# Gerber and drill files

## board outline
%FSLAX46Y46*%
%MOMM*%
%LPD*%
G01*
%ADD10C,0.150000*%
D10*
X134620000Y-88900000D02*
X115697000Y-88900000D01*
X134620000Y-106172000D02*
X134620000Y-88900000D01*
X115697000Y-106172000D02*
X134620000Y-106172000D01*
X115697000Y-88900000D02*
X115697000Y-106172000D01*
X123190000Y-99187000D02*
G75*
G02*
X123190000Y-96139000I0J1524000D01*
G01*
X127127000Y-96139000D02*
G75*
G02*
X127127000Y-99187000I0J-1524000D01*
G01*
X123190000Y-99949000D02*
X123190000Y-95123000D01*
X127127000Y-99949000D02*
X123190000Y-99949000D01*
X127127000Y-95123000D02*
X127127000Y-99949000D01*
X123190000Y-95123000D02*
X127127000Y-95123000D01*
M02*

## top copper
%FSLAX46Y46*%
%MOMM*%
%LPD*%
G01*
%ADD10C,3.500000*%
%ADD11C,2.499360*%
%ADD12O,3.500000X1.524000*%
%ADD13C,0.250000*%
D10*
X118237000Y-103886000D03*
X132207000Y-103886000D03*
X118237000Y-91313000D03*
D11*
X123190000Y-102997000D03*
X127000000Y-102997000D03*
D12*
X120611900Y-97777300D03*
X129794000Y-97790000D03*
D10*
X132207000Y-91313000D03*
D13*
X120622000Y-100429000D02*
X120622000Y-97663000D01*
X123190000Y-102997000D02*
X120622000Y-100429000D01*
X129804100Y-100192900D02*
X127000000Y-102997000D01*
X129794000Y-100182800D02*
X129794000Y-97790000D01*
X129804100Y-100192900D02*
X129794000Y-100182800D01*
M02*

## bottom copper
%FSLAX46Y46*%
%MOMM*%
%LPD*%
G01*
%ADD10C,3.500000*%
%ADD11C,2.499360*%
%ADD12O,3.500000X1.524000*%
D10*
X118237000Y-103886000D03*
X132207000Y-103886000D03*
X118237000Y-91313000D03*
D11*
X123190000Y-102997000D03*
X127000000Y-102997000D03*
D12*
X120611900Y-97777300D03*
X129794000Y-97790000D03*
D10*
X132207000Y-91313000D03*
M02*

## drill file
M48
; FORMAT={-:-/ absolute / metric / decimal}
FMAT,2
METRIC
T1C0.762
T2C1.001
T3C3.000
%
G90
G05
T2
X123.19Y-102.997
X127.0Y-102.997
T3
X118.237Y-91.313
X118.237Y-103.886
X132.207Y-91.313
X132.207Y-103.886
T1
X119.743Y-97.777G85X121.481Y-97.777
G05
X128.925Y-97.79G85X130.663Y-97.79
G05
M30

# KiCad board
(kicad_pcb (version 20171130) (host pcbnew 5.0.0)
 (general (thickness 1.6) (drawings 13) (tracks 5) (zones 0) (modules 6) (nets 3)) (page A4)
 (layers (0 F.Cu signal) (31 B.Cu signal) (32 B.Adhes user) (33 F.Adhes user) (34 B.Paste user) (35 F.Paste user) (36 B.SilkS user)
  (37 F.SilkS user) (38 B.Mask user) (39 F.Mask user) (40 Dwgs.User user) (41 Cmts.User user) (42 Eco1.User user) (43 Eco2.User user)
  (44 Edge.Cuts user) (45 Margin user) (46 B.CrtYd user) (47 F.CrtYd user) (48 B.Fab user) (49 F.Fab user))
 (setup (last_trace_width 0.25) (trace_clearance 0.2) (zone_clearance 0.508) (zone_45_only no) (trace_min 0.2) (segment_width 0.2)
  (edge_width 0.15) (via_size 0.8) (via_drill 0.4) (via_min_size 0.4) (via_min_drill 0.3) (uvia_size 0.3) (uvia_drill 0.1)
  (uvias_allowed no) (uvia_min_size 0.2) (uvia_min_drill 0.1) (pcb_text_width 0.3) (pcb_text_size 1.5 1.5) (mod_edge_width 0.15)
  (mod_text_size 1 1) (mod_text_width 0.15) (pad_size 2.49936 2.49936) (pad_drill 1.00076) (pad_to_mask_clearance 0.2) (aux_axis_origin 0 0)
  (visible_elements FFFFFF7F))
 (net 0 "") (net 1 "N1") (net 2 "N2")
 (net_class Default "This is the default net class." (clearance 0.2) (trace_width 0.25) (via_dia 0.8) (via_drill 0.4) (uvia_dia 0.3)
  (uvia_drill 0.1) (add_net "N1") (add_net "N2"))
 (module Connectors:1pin (layer F.Cu) (at 118.237 103.886)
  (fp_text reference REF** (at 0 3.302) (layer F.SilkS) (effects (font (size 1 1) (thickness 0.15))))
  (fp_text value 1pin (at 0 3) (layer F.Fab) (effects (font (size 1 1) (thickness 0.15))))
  (pad 1 thru_hole circle (at 0 0) (size 3.5 3.5) (drill 3) (layers *.Cu *.Mask)))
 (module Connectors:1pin (layer F.Cu) (at 132.207 103.886)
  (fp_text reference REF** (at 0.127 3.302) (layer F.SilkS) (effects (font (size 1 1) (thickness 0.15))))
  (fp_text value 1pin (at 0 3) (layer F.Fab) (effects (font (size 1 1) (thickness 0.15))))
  (pad 1 thru_hole circle (at 0 0) (size 3.5 3.5) (drill 3) (layers *.Cu *.Mask)))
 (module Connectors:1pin (layer F.Cu) (at 118.237 91.313)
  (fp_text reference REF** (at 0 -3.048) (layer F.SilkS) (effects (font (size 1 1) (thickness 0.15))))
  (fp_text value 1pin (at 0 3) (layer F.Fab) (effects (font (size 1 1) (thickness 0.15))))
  (pad 1 thru_hole circle (at 0 0) (size 3.5 3.5) (drill 3) (layers *.Cu *.Mask)))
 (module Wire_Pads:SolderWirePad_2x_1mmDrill (layer F.Cu) (at 125.095 102.997)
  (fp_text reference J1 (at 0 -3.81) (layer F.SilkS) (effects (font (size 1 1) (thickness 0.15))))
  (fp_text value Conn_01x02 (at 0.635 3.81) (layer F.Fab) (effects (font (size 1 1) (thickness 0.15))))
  (pad 1 thru_hole circle (at -1.905 0) (size 2.49936 2.49936) (drill 1.00076) (layers *.Cu *.Mask) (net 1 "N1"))
  (pad 1 thru_hole circle (at 1.905 0) (size 2.49936 2.49936) (drill 1.00076) (layers *.Cu *.Mask) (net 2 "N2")))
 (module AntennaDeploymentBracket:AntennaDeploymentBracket (layer F.Cu) (at 125.3744 97.7519)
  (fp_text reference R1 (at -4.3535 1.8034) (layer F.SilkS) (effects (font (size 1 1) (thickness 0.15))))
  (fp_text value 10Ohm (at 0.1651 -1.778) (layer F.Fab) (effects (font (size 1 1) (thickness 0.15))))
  (pad 1 thru_hole oval (at -4.7625 0.0254) (size 3.5 1.524) (drill oval 2.5 0.762) (layers *.Cu *.Mask) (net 1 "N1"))
  (pad 2 thru_hole oval (at 4.4196 0.0381) (size 3.5 1.524) (drill oval 2.5 0.762) (layers *.Cu *.Mask) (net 2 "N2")))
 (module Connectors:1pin (layer F.Cu) (at 132.207 91.313)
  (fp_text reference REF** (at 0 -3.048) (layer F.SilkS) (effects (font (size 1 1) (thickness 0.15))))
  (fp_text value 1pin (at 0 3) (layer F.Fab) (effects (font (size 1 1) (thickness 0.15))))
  (pad 1 thru_hole circle (at 0 0) (size 3.5 3.5) (drill 3) (layers *.Cu *.Mask)))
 (gr_line (start 134.62 88.9) (end 115.697 88.9) (layer Edge.Cuts) (width 0.15))
 (gr_line (start 134.62 106.172) (end 134.62 88.9) (layer Edge.Cuts) (width 0.15))
 (gr_line (start 115.697 106.172) (end 134.62 106.172) (layer Edge.Cuts) (width 0.15))
 (gr_line (start 115.697 88.9) (end 115.697 106.172) (layer Edge.Cuts) (width 0.15))
 (gr_arc (start 123.19 97.663) (end 123.19 96.139) (angle -180) (layer Edge.Cuts) (width 0.15))
 (gr_arc (start 127.127 97.663) (end 127.127 99.187) (angle -180) (layer Edge.Cuts) (width 0.15))
 (gr_line (start 123.19 99.949) (end 123.19 95.123) (layer Edge.Cuts) (width 0.15))
 (gr_line (start 127.127 99.949) (end 123.19 99.949) (layer Edge.Cuts) (width 0.15))
 (gr_line (start 127.127 95.123) (end 127.127 99.949) (layer Edge.Cuts) (width 0.15))
 (gr_line (start 123.19 95.123) (end 127.127 95.123) (layer Edge.Cuts) (width 0.15))
 (segment (start 120.622 100.429) (end 120.622 97.663) (width 0.25) (layer F.Cu) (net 1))
 (segment (start 123.19 102.997) (end 120.622 100.429) (width 0.25) (layer F.Cu) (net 1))
 (segment (start 129.8041 100.1929) (end 127 102.997) (width 0.25) (layer F.Cu) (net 2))
 (segment (start 129.794 100.1828) (end 129.794 97.79) (width 0.25) (layer F.Cu) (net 2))
 (segment (start 129.8041 100.1929) (end 129.794 100.1828) (width 0.25) (layer F.Cu) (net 2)))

